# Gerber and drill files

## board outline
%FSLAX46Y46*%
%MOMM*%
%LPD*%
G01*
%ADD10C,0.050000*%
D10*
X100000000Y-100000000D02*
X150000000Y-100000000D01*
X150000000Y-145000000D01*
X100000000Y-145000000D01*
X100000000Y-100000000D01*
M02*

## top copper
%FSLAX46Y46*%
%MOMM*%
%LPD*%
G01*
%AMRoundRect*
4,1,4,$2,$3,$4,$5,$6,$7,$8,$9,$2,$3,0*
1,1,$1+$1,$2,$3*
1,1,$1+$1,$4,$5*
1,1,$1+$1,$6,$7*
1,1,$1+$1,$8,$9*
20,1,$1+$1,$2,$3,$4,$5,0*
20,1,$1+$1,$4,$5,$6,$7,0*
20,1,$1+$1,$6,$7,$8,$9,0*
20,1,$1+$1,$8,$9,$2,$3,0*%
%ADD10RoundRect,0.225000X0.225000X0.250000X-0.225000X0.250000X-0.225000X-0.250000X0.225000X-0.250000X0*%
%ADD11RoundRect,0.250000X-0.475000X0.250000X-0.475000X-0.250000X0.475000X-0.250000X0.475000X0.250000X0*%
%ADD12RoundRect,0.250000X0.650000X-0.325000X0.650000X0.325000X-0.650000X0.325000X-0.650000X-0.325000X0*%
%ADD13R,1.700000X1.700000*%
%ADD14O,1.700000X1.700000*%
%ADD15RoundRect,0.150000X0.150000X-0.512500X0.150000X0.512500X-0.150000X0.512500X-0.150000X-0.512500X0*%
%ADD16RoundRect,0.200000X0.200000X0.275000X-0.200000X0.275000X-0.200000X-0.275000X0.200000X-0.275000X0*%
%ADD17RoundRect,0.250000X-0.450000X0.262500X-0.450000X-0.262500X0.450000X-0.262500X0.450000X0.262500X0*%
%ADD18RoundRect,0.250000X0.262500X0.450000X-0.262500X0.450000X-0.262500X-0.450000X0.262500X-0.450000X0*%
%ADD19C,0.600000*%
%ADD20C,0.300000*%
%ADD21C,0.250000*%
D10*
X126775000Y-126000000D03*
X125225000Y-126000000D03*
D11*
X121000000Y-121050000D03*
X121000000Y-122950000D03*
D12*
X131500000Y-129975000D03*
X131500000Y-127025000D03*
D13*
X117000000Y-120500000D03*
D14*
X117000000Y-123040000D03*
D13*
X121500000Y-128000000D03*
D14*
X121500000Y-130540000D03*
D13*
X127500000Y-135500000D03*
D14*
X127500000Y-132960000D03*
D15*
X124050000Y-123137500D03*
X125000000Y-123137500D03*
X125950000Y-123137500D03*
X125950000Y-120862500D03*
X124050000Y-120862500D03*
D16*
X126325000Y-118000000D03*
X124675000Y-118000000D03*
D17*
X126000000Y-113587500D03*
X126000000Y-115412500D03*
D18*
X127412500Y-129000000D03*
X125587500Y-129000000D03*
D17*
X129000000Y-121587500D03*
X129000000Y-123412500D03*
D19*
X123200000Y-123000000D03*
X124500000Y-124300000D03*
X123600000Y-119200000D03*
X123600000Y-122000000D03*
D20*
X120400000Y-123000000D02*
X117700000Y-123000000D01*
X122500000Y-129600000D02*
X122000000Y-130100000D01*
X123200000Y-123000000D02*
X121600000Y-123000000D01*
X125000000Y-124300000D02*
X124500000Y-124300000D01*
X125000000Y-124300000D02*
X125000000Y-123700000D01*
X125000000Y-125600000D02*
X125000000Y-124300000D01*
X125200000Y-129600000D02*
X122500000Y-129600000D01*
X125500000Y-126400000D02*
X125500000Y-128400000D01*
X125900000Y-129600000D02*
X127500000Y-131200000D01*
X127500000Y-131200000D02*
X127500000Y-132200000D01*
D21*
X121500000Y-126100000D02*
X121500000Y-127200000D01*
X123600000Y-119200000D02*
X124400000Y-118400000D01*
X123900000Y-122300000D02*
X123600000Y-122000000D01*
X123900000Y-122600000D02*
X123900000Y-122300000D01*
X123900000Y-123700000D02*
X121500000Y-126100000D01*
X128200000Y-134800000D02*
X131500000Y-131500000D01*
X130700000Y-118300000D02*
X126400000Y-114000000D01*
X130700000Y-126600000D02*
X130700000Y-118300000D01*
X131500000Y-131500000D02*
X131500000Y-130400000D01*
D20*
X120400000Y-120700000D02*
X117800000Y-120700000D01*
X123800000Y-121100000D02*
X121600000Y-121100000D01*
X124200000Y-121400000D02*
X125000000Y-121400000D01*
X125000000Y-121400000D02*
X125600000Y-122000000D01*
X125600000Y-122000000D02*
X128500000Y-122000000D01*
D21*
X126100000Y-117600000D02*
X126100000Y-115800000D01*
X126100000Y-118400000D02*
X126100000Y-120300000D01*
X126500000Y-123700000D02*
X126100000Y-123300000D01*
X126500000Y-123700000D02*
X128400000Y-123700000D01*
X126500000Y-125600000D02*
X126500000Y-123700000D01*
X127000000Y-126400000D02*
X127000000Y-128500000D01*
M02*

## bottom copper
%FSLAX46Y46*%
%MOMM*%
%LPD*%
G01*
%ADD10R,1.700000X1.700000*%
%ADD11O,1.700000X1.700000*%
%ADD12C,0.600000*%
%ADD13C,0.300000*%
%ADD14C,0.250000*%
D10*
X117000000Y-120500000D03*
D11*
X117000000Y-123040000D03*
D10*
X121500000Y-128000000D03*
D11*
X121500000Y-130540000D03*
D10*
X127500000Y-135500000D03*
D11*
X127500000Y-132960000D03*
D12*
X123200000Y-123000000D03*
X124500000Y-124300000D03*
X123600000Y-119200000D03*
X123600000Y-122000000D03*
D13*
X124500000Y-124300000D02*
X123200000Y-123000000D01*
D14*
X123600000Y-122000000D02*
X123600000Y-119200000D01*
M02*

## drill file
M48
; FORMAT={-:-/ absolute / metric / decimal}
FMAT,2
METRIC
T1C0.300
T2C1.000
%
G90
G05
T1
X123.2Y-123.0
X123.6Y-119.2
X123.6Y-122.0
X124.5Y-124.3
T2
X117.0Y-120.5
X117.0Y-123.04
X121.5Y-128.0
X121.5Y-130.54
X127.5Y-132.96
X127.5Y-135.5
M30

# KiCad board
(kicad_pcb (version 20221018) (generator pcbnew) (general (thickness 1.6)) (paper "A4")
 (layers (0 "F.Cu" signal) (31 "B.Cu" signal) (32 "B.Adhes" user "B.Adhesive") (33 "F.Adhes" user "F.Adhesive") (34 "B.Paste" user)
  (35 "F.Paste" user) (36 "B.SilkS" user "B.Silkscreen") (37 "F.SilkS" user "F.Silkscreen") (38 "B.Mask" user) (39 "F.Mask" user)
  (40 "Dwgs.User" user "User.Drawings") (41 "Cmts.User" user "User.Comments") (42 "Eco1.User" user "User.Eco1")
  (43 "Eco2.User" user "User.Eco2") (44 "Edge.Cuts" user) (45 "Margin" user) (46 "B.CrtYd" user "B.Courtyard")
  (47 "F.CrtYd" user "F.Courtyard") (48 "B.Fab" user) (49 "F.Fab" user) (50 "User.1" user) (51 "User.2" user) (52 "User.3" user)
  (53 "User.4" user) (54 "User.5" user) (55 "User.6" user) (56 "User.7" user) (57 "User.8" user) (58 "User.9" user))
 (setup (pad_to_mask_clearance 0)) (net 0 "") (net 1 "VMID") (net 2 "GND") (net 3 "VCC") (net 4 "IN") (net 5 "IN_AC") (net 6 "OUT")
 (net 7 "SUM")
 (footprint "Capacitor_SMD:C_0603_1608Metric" (layer "F.Cu") (at 126 126 180)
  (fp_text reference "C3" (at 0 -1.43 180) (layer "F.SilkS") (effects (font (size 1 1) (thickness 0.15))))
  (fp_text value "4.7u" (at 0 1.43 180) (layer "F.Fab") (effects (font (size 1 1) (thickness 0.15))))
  (pad "1" smd roundrect (at -0.775 0 180) (size 0.9 0.95) (layers "F.Cu" "F.Paste" "F.Mask") (roundrect_rratio 0.25) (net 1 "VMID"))
  (pad "2" smd roundrect (at 0.775 0 180) (size 0.9 0.95) (layers "F.Cu" "F.Paste" "F.Mask") (roundrect_rratio 0.25) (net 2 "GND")))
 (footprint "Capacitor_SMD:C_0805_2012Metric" (layer "F.Cu") (at 121 122 -90)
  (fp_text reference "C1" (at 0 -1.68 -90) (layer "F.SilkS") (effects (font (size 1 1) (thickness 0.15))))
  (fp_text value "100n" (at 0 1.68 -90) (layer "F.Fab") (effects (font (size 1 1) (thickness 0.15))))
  (pad "1" smd roundrect (at -0.95 0 270) (size 1 1.45) (layers "F.Cu" "F.Paste" "F.Mask") (roundrect_rratio 0.25) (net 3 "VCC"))
  (pad "2" smd roundrect (at 0.95 0 270) (size 1 1.45) (layers "F.Cu" "F.Paste" "F.Mask") (roundrect_rratio 0.25) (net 2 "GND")))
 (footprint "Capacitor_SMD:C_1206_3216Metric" (layer "F.Cu") (at 131.5 128.5 90)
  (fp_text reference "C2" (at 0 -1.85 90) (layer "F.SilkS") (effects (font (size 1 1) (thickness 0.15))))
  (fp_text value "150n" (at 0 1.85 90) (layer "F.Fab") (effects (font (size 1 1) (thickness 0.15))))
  (pad "1" smd roundrect (at -1.475 0 90) (size 1.15 1.8) (layers "F.Cu" "F.Paste" "F.Mask") (roundrect_rratio 0.217391) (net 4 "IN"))
  (pad "2" smd roundrect (at 1.475 0 90) (size 1.15 1.8) (layers "F.Cu" "F.Paste" "F.Mask") (roundrect_rratio 0.217391) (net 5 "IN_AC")))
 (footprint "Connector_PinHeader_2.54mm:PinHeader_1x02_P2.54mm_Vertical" (layer "F.Cu") (at 117 120.5)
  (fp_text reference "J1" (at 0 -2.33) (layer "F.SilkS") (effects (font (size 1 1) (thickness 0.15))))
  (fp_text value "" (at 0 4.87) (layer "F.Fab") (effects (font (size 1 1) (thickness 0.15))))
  (pad "1" thru_hole rect (at 0 0) (size 1.7 1.7) (drill 1) (layers "*.Cu" "*.Mask") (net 3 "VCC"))
  (pad "2" thru_hole oval (at 0 2.54) (size 1.7 1.7) (drill 1) (layers "*.Cu" "*.Mask") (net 2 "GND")))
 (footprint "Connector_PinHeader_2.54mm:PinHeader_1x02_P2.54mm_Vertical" (layer "F.Cu") (at 121.5 128)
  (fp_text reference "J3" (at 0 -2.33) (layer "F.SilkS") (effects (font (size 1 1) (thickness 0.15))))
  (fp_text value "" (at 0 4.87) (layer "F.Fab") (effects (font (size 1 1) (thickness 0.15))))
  (pad "1" thru_hole rect (at 0 0) (size 1.7 1.7) (drill 1) (layers "*.Cu" "*.Mask") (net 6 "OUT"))
  (pad "2" thru_hole oval (at 0 2.54) (size 1.7 1.7) (drill 1) (layers "*.Cu" "*.Mask") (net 2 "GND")))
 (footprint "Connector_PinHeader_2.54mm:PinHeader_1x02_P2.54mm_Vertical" (layer "F.Cu") (at 127.5 135.5 180)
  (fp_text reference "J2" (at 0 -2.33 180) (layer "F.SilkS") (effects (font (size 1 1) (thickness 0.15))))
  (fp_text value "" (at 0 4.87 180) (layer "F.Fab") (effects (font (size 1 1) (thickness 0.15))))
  (pad "1" thru_hole rect (at 0 0 180) (size 1.7 1.7) (drill 1) (layers "*.Cu" "*.Mask") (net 4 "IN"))
  (pad "2" thru_hole oval (at 0 2.54 180) (size 1.7 1.7) (drill 1) (layers "*.Cu" "*.Mask") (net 2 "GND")))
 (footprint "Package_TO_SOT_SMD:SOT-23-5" (layer "F.Cu") (at 125 122 90)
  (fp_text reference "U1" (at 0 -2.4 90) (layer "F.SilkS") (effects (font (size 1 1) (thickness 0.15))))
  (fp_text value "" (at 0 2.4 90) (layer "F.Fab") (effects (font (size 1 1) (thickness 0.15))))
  (pad "1" smd roundrect (at -1.1375 -0.95 90) (size 1.325 0.6) (layers "F.Cu" "F.Paste" "F.Mask") (roundrect_rratio 0.25) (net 6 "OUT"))
  (pad "2" smd roundrect (at -1.1375 0 90) (size 1.325 0.6) (layers "F.Cu" "F.Paste" "F.Mask") (roundrect_rratio 0.25) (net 2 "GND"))
  (pad "3" smd roundrect (at -1.1375 0.95 90) (size 1.325 0.6) (layers "F.Cu" "F.Paste" "F.Mask") (roundrect_rratio 0.25) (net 1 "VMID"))
  (pad "4" smd roundrect (at 1.1375 0.95 90) (size 1.325 0.6) (layers "F.Cu" "F.Paste" "F.Mask") (roundrect_rratio 0.25) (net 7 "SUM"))
  (pad "5" smd roundrect (at 1.1375 -0.95 90) (size 1.325 0.6) (layers "F.Cu" "F.Paste" "F.Mask") (roundrect_rratio 0.25) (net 3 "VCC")))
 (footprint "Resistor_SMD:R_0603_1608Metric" (layer "F.Cu") (at 125.5 118 180)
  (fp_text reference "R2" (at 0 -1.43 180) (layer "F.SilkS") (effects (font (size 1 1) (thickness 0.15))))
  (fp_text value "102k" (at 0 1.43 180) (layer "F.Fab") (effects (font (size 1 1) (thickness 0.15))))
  (pad "1" smd roundrect (at -0.825 0 180) (size 0.8 0.95) (layers "F.Cu" "F.Paste" "F.Mask") (roundrect_rratio 0.25) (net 7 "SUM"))
  (pad "2" smd roundrect (at 0.825 0 180) (size 0.8 0.95) (layers "F.Cu" "F.Paste" "F.Mask") (roundrect_rratio 0.25) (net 6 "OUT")))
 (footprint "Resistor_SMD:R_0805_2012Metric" (layer "F.Cu") (at 126 114.5 -90)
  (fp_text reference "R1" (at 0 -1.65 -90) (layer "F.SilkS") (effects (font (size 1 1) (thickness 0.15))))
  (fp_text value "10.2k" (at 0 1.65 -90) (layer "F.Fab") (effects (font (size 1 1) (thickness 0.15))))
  (pad "1" smd roundrect (at -0.9125 0 270) (size 1.025 1.4) (layers "F.Cu" "F.Paste" "F.Mask") (roundrect_rratio 0.243902) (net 5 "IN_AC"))
  (pad "2" smd roundrect (at 0.9125 0 270) (size 1.025 1.4) (layers "F.Cu" "F.Paste" "F.Mask") (roundrect_rratio 0.243902) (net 7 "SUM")))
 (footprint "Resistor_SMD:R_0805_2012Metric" (layer "F.Cu") (at 126.5 129 180)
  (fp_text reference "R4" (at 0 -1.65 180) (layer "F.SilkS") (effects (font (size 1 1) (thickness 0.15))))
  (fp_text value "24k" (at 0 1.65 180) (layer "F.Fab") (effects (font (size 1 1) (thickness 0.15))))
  (pad "1" smd roundrect (at -0.9125 0 180) (size 1.025 1.4) (layers "F.Cu" "F.Paste" "F.Mask") (roundrect_rratio 0.243902) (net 1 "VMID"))
  (pad "2" smd roundrect (at 0.9125 0 180) (size 1.025 1.4) (layers "F.Cu" "F.Paste" "F.Mask") (roundrect_rratio 0.243902) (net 2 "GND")))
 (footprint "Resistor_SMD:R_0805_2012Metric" (layer "F.Cu") (at 129 122.5 -90)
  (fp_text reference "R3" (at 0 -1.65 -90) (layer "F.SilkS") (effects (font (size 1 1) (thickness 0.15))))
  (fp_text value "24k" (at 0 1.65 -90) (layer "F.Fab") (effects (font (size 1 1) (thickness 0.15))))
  (pad "1" smd roundrect (at -0.9125 0 270) (size 1.025 1.4) (layers "F.Cu" "F.Paste" "F.Mask") (roundrect_rratio 0.243902) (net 3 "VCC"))
  (pad "2" smd roundrect (at 0.9125 0 270) (size 1.025 1.4) (layers "F.Cu" "F.Paste" "F.Mask") (roundrect_rratio 0.243902) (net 1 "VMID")))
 (gr_rect (start 100 100) (end 150 145) (stroke (width 0.05) (type default)) (fill none) (layer "Edge.Cuts"))
 (segment (start 120.4 123) (end 117.7 123) (width 0.3) (layer "F.Cu") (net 2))
 (segment (start 122.5 129.6) (end 122 130.1) (width 0.3) (layer "F.Cu") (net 2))
 (segment (start 123.2 123) (end 121.6 123) (width 0.3) (layer "F.Cu") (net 2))
 (segment (start 125 124.3) (end 124.5 124.3) (width 0.3) (layer "F.Cu") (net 2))
 (segment (start 125 124.3) (end 125 123.7) (width 0.3) (layer "F.Cu") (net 2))
 (segment (start 125 125.6) (end 125 124.3) (width 0.3) (layer "F.Cu") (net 2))
 (segment (start 125.2 129.6) (end 122.5 129.6) (width 0.3) (layer "F.Cu") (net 2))
 (segment (start 125.5 126.4) (end 125.5 128.4) (width 0.3) (layer "F.Cu") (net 2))
 (segment (start 125.9 129.6) (end 127.5 131.2) (width 0.3) (layer "F.Cu") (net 2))
 (segment (start 127.5 131.2) (end 127.5 132.2) (width 0.3) (layer "F.Cu") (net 2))
 (via (at 123.2 123) (size 0.6) (drill 0.3) (layers "F.Cu" "B.Cu") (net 2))
 (via (at 124.5 124.3) (size 0.6) (drill 0.3) (layers "F.Cu" "B.Cu") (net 2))
 (segment (start 121.5 126.1) (end 121.5 127.2) (width 0.25) (layer "F.Cu") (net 6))
 (segment (start 123.6 119.2) (end 124.4 118.4) (width 0.25) (layer "F.Cu") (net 6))
 (segment (start 123.9 122.3) (end 123.6 122) (width 0.25) (layer "F.Cu") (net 6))
 (segment (start 123.9 122.6) (end 123.9 122.3) (width 0.25) (layer "F.Cu") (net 6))
 (segment (start 123.9 123.7) (end 121.5 126.1) (width 0.25) (layer "F.Cu") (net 6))
 (segment (start 124.5 124.3) (end 123.2 123) (width 0.3) (layer "B.Cu") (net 2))
 (segment (start 128.2 134.8) (end 131.5 131.5) (width 0.25) (layer "F.Cu") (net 4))
 (segment (start 130.7 118.3) (end 126.4 114) (width 0.25) (layer "F.Cu") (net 5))
 (segment (start 130.7 126.6) (end 130.7 118.3) (width 0.25) (layer "F.Cu") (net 5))
 (segment (start 131.5 131.5) (end 131.5 130.4) (width 0.25) (layer "F.Cu") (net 4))
 (via (at 123.6 119.2) (size 0.6) (drill 0.3) (layers "F.Cu" "B.Cu") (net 6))
 (via (at 123.6 122) (size 0.6) (drill 0.3) (layers "F.Cu" "B.Cu") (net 6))
 (segment (start 120.4 120.7) (end 117.8 120.7) (width 0.3) (layer "F.Cu") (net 3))
 (segment (start 123.6 122) (end 123.6 119.2) (width 0.25) (layer "B.Cu") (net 6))
 (segment (start 123.8 121.1) (end 121.6 121.1) (width 0.3) (layer "F.Cu") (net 3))
 (segment (start 124.2 121.4) (end 125 121.4) (width 0.3) (layer "F.Cu") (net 3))
 (segment (start 125 121.4) (end 125.6 122) (width 0.3) (layer "F.Cu") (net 3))
 (segment (start 125.6 122) (end 128.5 122) (width 0.3) (layer "F.Cu") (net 3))
 (segment (start 126.1 117.6) (end 126.1 115.8) (width 0.25) (layer "F.Cu") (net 7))
 (segment (start 126.1 118.4) (end 126.1 120.3) (width 0.25) (layer "F.Cu") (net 7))
 (segment (start 126.5 123.7) (end 126.1 123.3) (width 0.25) (layer "F.Cu") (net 1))
 (segment (start 126.5 123.7) (end 128.4 123.7) (width 0.25) (layer "F.Cu") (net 1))
 (segment (start 126.5 125.6) (end 126.5 123.7) (width 0.25) (layer "F.Cu") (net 1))
 (segment (start 127 126.4) (end 127 128.5) (width 0.25) (layer "F.Cu") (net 1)))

